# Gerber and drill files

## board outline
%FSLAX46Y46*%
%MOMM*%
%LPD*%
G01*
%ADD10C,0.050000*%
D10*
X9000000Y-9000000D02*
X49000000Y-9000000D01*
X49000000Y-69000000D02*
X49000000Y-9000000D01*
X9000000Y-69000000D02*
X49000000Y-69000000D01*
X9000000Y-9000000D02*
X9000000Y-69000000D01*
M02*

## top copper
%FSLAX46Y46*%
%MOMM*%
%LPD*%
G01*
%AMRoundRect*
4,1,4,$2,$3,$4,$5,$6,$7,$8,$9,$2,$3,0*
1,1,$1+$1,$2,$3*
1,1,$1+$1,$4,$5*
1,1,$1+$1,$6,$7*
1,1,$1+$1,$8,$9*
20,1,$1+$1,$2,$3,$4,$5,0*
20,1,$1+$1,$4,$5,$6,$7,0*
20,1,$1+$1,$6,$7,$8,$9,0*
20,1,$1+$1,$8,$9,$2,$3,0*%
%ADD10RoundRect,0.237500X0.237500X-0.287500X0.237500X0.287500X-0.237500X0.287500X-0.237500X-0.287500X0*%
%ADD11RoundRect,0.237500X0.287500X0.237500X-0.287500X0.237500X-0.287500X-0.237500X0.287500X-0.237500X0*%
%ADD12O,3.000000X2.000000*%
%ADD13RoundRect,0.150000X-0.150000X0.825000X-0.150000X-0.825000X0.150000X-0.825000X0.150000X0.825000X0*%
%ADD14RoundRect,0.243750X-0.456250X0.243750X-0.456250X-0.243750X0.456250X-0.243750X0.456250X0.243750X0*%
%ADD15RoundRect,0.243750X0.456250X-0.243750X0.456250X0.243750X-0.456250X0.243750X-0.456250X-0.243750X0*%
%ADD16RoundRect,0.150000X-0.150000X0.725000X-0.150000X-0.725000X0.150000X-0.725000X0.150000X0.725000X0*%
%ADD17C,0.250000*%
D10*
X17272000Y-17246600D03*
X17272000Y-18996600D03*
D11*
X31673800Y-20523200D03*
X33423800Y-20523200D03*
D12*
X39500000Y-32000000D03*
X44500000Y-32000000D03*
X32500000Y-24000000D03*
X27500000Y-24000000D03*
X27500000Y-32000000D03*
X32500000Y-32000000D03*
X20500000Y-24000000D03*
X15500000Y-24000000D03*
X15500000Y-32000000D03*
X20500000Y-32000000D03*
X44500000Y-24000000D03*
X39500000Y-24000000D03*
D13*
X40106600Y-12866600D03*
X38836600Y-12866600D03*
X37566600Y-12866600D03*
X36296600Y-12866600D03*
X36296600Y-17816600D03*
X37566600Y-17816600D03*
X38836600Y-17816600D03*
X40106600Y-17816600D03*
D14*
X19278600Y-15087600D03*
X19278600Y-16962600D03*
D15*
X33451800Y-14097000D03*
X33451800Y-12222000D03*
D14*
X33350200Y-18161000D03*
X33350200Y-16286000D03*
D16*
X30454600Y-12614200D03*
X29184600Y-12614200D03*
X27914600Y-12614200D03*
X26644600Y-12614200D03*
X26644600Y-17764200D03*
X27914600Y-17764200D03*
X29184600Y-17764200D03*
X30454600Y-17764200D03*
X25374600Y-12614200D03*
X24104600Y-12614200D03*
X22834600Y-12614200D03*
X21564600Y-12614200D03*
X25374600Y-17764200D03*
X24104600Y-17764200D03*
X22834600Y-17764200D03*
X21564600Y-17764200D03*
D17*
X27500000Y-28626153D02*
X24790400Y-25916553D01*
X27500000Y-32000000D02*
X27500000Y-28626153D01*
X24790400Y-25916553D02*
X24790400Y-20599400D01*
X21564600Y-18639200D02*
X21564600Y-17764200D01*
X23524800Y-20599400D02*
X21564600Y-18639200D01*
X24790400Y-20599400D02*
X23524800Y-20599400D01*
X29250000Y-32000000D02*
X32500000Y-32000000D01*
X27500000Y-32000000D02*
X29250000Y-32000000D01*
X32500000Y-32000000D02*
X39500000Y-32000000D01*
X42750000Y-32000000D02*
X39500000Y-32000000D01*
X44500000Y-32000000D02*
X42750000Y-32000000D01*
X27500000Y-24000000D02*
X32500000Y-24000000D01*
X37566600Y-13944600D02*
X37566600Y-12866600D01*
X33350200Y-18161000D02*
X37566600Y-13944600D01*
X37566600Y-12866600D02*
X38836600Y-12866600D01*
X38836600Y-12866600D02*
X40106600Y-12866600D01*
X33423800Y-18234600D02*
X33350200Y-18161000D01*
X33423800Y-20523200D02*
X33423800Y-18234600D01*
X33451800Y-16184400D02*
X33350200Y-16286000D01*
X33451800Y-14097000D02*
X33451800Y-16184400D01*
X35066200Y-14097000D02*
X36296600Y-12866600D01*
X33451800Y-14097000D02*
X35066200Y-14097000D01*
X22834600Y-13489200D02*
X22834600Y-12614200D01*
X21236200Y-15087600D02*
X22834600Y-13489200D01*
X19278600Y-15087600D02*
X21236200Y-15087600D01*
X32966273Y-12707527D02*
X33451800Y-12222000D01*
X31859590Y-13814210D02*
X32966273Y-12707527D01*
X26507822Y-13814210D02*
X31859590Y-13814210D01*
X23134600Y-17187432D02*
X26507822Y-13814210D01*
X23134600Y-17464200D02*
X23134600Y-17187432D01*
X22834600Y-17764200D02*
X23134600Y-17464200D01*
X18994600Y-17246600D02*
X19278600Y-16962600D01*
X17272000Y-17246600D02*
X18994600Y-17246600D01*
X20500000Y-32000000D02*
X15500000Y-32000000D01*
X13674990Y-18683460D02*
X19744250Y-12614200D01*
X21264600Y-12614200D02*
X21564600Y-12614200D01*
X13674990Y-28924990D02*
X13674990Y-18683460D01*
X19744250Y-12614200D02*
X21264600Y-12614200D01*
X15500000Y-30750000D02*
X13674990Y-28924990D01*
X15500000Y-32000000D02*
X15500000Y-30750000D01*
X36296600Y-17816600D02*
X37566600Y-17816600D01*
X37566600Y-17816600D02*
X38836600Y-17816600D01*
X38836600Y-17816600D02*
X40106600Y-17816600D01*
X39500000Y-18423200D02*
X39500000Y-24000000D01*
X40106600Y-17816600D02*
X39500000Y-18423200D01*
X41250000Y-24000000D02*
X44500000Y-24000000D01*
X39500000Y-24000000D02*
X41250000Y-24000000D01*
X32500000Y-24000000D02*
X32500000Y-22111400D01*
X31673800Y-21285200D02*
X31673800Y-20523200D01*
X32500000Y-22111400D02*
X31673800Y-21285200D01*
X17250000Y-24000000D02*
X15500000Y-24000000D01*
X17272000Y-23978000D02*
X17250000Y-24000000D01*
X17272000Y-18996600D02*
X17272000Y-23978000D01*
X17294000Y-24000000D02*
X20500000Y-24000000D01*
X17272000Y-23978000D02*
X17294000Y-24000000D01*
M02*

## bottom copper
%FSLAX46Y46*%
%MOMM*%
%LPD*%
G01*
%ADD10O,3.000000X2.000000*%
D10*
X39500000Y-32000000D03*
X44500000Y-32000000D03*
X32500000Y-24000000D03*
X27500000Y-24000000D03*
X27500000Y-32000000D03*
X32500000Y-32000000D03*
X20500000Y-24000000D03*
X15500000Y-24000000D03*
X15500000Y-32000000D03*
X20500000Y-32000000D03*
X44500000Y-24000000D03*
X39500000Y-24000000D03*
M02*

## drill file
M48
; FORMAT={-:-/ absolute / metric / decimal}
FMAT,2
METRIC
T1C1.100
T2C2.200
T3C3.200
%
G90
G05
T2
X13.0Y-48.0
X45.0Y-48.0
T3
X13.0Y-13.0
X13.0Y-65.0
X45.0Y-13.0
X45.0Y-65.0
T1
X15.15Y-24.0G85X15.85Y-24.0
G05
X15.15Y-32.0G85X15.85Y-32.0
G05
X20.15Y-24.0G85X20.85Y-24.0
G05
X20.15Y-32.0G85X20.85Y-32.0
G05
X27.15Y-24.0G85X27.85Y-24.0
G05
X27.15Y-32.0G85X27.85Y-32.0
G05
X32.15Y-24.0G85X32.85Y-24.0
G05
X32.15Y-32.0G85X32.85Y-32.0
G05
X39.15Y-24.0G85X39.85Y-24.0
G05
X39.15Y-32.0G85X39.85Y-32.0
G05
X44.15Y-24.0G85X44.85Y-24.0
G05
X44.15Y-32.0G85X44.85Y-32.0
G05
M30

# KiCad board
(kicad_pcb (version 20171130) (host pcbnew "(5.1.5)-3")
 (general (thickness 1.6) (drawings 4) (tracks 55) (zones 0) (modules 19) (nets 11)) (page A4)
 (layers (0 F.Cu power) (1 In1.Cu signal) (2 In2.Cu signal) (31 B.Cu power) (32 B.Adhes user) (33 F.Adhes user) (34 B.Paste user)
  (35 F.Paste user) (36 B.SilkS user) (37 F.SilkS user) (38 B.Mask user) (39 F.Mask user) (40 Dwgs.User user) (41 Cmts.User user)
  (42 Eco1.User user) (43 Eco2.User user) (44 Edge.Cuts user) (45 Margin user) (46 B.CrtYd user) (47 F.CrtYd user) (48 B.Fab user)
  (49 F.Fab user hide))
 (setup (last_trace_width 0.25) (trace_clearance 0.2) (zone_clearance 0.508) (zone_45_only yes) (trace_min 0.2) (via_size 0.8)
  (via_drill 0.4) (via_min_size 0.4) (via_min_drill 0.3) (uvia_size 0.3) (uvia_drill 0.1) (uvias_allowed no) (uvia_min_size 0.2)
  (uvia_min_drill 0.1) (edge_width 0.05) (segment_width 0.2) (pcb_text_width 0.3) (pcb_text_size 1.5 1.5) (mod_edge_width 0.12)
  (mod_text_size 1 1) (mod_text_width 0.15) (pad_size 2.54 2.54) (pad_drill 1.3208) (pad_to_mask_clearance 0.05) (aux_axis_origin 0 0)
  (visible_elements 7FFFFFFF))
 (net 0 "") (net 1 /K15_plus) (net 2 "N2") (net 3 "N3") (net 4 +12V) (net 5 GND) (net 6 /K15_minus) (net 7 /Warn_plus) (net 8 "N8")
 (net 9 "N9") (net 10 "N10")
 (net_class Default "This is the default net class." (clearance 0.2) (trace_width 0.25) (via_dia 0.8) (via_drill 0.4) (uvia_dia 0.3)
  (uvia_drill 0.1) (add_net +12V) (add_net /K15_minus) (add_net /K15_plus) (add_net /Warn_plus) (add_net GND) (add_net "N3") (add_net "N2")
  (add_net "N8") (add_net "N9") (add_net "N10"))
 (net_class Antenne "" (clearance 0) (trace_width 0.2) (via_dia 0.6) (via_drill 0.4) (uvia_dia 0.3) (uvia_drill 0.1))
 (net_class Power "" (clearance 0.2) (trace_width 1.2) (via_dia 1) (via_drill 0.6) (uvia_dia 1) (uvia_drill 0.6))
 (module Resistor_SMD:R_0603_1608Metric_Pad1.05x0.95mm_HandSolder (layer F.Cu) (at 17.272 18.1216 90)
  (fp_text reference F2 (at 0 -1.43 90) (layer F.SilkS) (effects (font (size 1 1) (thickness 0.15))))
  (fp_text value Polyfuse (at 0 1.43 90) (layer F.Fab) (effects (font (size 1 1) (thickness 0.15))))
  (pad 2 smd roundrect (at 0.875 0 90) (size 1.05 0.95) (layers F.Cu F.Paste F.Mask) (roundrect_rratio 0.25) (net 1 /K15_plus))
  (pad 1 smd roundrect (at -0.875 0 90) (size 1.05 0.95) (layers F.Cu F.Paste F.Mask) (roundrect_rratio 0.25) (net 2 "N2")))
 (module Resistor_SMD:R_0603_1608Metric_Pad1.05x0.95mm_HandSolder (layer F.Cu) (at 32.5488 20.5232 180)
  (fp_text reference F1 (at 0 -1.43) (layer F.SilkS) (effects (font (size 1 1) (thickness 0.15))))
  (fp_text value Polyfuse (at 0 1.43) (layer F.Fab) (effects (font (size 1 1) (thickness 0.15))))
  (pad 2 smd roundrect (at 0.875 0 180) (size 1.05 0.95) (layers F.Cu F.Paste F.Mask) (roundrect_rratio 0.25) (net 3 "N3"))
  (pad 1 smd roundrect (at -0.875 0 180) (size 1.05 0.95) (layers F.Cu F.Paste F.Mask) (roundrect_rratio 0.25) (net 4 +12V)))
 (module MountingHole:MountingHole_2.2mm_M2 (layer F.Cu) (at 45 48)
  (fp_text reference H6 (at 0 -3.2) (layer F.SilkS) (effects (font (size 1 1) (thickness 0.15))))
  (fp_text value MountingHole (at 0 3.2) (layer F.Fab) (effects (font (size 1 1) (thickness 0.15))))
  (pad 1 np_thru_hole circle (at 0 0) (size 2.2 2.2) (drill 2.2) (layers *.Cu *.Mask)))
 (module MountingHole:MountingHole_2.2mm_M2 (layer F.Cu) (at 13 48)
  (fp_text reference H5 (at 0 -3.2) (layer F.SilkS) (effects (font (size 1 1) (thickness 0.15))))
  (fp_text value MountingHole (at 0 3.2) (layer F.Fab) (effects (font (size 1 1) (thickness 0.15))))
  (pad 1 np_thru_hole circle (at 0 0) (size 2.2 2.2) (drill 2.2) (layers *.Cu *.Mask)))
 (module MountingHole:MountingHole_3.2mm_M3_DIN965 (layer F.Cu) (at 13 13)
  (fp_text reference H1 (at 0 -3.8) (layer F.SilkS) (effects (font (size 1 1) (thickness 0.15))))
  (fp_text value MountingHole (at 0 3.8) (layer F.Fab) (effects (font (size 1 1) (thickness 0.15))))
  (pad 1 np_thru_hole circle (at 0 0) (size 3.2 3.2) (drill 3.2) (layers *.Cu *.Mask)))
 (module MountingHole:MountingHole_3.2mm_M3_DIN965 (layer F.Cu) (at 13 65)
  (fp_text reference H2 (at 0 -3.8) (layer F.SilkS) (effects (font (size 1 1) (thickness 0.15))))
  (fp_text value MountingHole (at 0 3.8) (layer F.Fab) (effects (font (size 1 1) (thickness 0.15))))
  (pad 1 np_thru_hole circle (at 0 0) (size 3.2 3.2) (drill 3.2) (layers *.Cu *.Mask)))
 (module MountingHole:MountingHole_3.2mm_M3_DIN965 (layer F.Cu) (at 45 13)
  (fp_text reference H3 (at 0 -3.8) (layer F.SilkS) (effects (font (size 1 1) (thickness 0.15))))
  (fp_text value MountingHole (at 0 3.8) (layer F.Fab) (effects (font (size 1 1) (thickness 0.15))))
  (pad 1 np_thru_hole circle (at 0 0) (size 3.2 3.2) (drill 3.2) (layers *.Cu *.Mask)))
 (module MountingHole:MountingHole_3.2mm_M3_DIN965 (layer F.Cu) (at 45 65)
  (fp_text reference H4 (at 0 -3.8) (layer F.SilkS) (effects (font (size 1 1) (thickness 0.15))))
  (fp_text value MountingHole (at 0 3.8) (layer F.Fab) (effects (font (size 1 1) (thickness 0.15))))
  (pad 1 np_thru_hole circle (at 0 0) (size 3.2 3.2) (drill 3.2) (layers *.Cu *.Mask)))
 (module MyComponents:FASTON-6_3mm (layer F.Cu) (at 42 32)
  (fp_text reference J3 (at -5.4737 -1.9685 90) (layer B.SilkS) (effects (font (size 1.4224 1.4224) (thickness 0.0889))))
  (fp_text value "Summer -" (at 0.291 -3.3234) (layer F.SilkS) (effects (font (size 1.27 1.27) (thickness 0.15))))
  (pad 1 thru_hole oval (at -2.5 0) (size 3 2) (drill oval 1.8 1.1) (layers *.Cu F.Paste F.SilkS F.Mask) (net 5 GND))
  (pad 1 thru_hole oval (at 2.5 0) (size 3 2) (drill oval 1.8 1.1) (layers *.Cu F.Paste F.SilkS F.Mask) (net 5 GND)))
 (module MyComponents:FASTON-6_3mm (layer F.Cu) (at 30 24)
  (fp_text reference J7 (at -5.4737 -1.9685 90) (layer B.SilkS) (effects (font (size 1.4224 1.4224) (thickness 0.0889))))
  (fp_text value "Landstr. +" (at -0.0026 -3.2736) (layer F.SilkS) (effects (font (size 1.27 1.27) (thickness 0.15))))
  (pad 1 thru_hole oval (at 2.5 0) (size 3 2) (drill oval 1.8 1.1) (layers *.Cu F.Paste F.SilkS F.Mask) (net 3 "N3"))
  (pad 1 thru_hole oval (at -2.5 0) (size 3 2) (drill oval 1.8 1.1) (layers *.Cu F.Paste F.SilkS F.Mask) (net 3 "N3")))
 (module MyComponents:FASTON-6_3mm (layer F.Cu) (at 30 32)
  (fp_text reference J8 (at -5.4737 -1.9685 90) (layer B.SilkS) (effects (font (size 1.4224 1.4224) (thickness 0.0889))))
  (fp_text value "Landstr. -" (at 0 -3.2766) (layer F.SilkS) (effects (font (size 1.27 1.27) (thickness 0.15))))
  (pad 1 thru_hole oval (at -2.5 0) (size 3 2) (drill oval 1.8 1.1) (layers *.Cu F.Paste F.SilkS F.Mask) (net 5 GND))
  (pad 1 thru_hole oval (at 2.5 0) (size 3 2) (drill oval 1.8 1.1) (layers *.Cu F.Paste F.SilkS F.Mask) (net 5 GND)))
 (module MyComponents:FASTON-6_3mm (layer F.Cu) (at 18 24)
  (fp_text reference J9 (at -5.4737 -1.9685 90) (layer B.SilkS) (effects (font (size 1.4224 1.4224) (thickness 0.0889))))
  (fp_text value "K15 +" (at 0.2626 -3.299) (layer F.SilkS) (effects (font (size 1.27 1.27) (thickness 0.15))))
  (pad 1 thru_hole oval (at 2.5 0) (size 3 2) (drill oval 1.8 1.1) (layers *.Cu F.Paste F.SilkS F.Mask) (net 2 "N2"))
  (pad 1 thru_hole oval (at -2.5 0) (size 3 2) (drill oval 1.8 1.1) (layers *.Cu F.Paste F.SilkS F.Mask) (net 2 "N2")))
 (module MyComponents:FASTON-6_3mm (layer F.Cu) (at 18 32)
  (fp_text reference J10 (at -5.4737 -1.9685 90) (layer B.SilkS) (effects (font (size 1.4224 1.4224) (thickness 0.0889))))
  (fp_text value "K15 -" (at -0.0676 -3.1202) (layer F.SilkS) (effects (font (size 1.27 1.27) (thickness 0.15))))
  (pad 1 thru_hole oval (at -2.5 0) (size 3 2) (drill oval 1.8 1.1) (layers *.Cu F.Paste F.SilkS F.Mask) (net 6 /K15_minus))
  (pad 1 thru_hole oval (at 2.5 0) (size 3 2) (drill oval 1.8 1.1) (layers *.Cu F.Paste F.SilkS F.Mask) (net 6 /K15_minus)))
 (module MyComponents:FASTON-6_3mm (layer F.Cu) (at 42 24)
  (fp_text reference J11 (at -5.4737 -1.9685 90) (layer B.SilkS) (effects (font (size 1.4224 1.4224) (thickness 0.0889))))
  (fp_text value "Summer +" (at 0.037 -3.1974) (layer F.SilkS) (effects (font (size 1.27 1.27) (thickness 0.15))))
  (pad 1 thru_hole oval (at 2.5 0) (size 3 2) (drill oval 1.8 1.1) (layers *.Cu F.Paste F.SilkS F.Mask) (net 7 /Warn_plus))
  (pad 1 thru_hole oval (at -2.5 0) (size 3 2) (drill oval 1.8 1.1) (layers *.Cu F.Paste F.SilkS F.Mask) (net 7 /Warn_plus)))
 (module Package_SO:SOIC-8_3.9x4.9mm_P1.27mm (layer F.Cu) (at 38.2016 15.3416 270)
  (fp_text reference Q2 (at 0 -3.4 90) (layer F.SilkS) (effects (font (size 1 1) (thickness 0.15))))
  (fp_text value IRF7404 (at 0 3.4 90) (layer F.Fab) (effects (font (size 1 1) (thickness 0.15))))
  (pad 1 smd roundrect (at -2.475 -1.905 270) (size 1.95 0.6) (layers F.Cu F.Paste F.Mask) (roundrect_rratio 0.25) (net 4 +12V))
  (pad 2 smd roundrect (at -2.475 -0.635 270) (size 1.95 0.6) (layers F.Cu F.Paste F.Mask) (roundrect_rratio 0.25) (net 4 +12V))
  (pad 3 smd roundrect (at -2.475 0.635 270) (size 1.95 0.6) (layers F.Cu F.Paste F.Mask) (roundrect_rratio 0.25) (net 4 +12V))
  (pad 4 smd roundrect (at -2.475 1.905 270) (size 1.95 0.6) (layers F.Cu F.Paste F.Mask) (roundrect_rratio 0.25) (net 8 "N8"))
  (pad 5 smd roundrect (at 2.475 1.905 270) (size 1.95 0.6) (layers F.Cu F.Paste F.Mask) (roundrect_rratio 0.25) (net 7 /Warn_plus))
  (pad 6 smd roundrect (at 2.475 0.635 270) (size 1.95 0.6) (layers F.Cu F.Paste F.Mask) (roundrect_rratio 0.25) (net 7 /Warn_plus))
  (pad 7 smd roundrect (at 2.475 -0.635 270) (size 1.95 0.6) (layers F.Cu F.Paste F.Mask) (roundrect_rratio 0.25) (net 7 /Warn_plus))
  (pad 8 smd roundrect (at 2.475 -1.905 270) (size 1.95 0.6) (layers F.Cu F.Paste F.Mask) (roundrect_rratio 0.25) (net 7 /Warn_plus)))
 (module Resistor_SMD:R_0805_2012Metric (layer F.Cu) (at 19.2786 16.0251 270)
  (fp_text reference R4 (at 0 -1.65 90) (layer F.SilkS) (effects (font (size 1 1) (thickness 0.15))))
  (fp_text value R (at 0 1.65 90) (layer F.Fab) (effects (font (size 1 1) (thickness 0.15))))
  (pad 1 smd roundrect (at -0.9375 0 270) (size 0.975 1.4) (layers F.Cu F.Paste F.Mask) (roundrect_rratio 0.25) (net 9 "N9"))
  (pad 2 smd roundrect (at 0.9375 0 270) (size 0.975 1.4) (layers F.Cu F.Paste F.Mask) (roundrect_rratio 0.25) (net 1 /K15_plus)))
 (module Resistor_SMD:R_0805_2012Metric (layer F.Cu) (at 33.4518 13.1595 90)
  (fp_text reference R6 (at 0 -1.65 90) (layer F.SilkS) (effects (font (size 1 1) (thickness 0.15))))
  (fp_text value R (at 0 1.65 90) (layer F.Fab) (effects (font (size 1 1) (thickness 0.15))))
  (pad 1 smd roundrect (at -0.9375 0 90) (size 0.975 1.4) (layers F.Cu F.Paste F.Mask) (roundrect_rratio 0.25) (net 8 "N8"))
  (pad 2 smd roundrect (at 0.9375 0 90) (size 0.975 1.4) (layers F.Cu F.Paste F.Mask) (roundrect_rratio 0.25) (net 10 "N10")))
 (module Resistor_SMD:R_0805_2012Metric (layer F.Cu) (at 33.3502 17.2235 270)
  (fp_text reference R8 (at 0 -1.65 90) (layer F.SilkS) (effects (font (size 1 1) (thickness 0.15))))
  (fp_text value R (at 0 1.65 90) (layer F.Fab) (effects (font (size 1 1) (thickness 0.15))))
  (pad 2 smd roundrect (at 0.9375 0 270) (size 0.975 1.4) (layers F.Cu F.Paste F.Mask) (roundrect_rratio 0.25) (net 4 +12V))
  (pad 1 smd roundrect (at -0.9375 0 270) (size 0.975 1.4) (layers F.Cu F.Paste F.Mask) (roundrect_rratio 0.25) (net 8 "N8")))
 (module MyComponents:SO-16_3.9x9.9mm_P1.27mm (layer F.Cu) (at 28.5496 15.1892 270)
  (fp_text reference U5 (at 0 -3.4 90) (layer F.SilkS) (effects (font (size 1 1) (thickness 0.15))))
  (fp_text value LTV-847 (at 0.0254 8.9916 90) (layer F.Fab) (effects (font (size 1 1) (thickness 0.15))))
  (pad 1 smd roundrect (at -2.575 -1.905 270) (size 1.75 0.6) (layers F.Cu F.Paste F.Mask) (roundrect_rratio 0.25))
  (pad 2 smd roundrect (at -2.575 -0.635 270) (size 1.75 0.6) (layers F.Cu F.Paste F.Mask) (roundrect_rratio 0.25))
  (pad 3 smd roundrect (at -2.575 0.635 270) (size 1.75 0.6) (layers F.Cu F.Paste F.Mask) (roundrect_rratio 0.25))
  (pad 4 smd roundrect (at -2.575 1.905 270) (size 1.75 0.6) (layers F.Cu F.Paste F.Mask) (roundrect_rratio 0.25))
  (pad 13 smd roundrect (at 2.575 1.905 270) (size 1.75 0.6) (layers F.Cu F.Paste F.Mask) (roundrect_rratio 0.25))
  (pad 14 smd roundrect (at 2.575 0.635 270) (size 1.75 0.6) (layers F.Cu F.Paste F.Mask) (roundrect_rratio 0.25))
  (pad 15 smd roundrect (at 2.575 -0.635 270) (size 1.75 0.6) (layers F.Cu F.Paste F.Mask) (roundrect_rratio 0.25))
  (pad 16 smd roundrect (at 2.575 -1.905 270) (size 1.75 0.6) (layers F.Cu F.Paste F.Mask) (roundrect_rratio 0.25))
  (pad 5 smd roundrect (at -2.575 3.175 270) (size 1.75 0.6) (layers F.Cu F.Paste F.Mask) (roundrect_rratio 0.25))
  (pad 6 smd roundrect (at -2.575 4.445 270) (size 1.75 0.6) (layers F.Cu F.Paste F.Mask) (roundrect_rratio 0.25))
  (pad 7 smd roundrect (at -2.575 5.715 270) (size 1.75 0.6) (layers F.Cu F.Paste F.Mask) (roundrect_rratio 0.25) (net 9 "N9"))
  (pad 8 smd roundrect (at -2.575 6.985 270) (size 1.75 0.6) (layers F.Cu F.Paste F.Mask) (roundrect_rratio 0.25) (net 6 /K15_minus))
  (pad 12 smd roundrect (at 2.575 3.175 270) (size 1.75 0.6) (layers F.Cu F.Paste F.Mask) (roundrect_rratio 0.25))
  (pad 11 smd roundrect (at 2.575 4.445 270) (size 1.75 0.6) (layers F.Cu F.Paste F.Mask) (roundrect_rratio 0.25))
  (pad 10 smd roundrect (at 2.575 5.715 270) (size 1.75 0.6) (layers F.Cu F.Paste F.Mask) (roundrect_rratio 0.25) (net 10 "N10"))
  (pad 9 smd roundrect (at 2.575 6.985 270) (size 1.75 0.6) (layers F.Cu F.Paste F.Mask) (roundrect_rratio 0.25) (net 5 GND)))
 (gr_line (start 9 9) (end 49 9) (layer Edge.Cuts) (width 0.05))
 (gr_line (start 49 69) (end 49 9) (layer Edge.Cuts) (width 0.05))
 (gr_line (start 9 69) (end 49 69) (layer Edge.Cuts) (width 0.05))
 (gr_line (start 9 9) (end 9 69) (layer Edge.Cuts) (width 0.05))
 (segment (start 27.5 28.626153) (end 24.7904 25.916553) (width 0.25) (layer F.Cu) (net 5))
 (segment (start 27.5 32) (end 27.5 28.626153) (width 0.25) (layer F.Cu) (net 5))
 (segment (start 24.7904 25.916553) (end 24.7904 20.5994) (width 0.25) (layer F.Cu) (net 5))
 (segment (start 21.5646 18.6392) (end 21.5646 17.7642) (width 0.25) (layer F.Cu) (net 5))
 (segment (start 23.5248 20.5994) (end 21.5646 18.6392) (width 0.25) (layer F.Cu) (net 5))
 (segment (start 24.7904 20.5994) (end 23.5248 20.5994) (width 0.25) (layer F.Cu) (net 5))
 (segment (start 29.25 32) (end 32.5 32) (width 0.25) (layer F.Cu) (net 5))
 (segment (start 27.5 32) (end 29.25 32) (width 0.25) (layer F.Cu) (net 5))
 (segment (start 32.5 32) (end 39.5 32) (width 0.25) (layer F.Cu) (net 5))
 (segment (start 42.75 32) (end 39.5 32) (width 0.25) (layer F.Cu) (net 5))
 (segment (start 44.5 32) (end 42.75 32) (width 0.25) (layer F.Cu) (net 5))
 (segment (start 27.5 24) (end 32.5 24) (width 0.25) (layer F.Cu) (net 3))
 (segment (start 37.5666 13.9446) (end 37.5666 12.8666) (width 0.25) (layer F.Cu) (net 4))
 (segment (start 33.3502 18.161) (end 37.5666 13.9446) (width 0.25) (layer F.Cu) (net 4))
 (segment (start 37.5666 12.8666) (end 38.8366 12.8666) (width 0.25) (layer F.Cu) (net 4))
 (segment (start 38.8366 12.8666) (end 40.1066 12.8666) (width 0.25) (layer F.Cu) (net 4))
 (segment (start 33.4238 18.2346) (end 33.3502 18.161) (width 0.25) (layer F.Cu) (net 4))
 (segment (start 33.4238 20.5232) (end 33.4238 18.2346) (width 0.25) (layer F.Cu) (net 4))
 (segment (start 33.4518 16.1844) (end 33.3502 16.286) (width 0.25) (layer F.Cu) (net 8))
 (segment (start 33.4518 14.097) (end 33.4518 16.1844) (width 0.25) (layer F.Cu) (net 8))
 (segment (start 35.0662 14.097) (end 36.2966 12.8666) (width 0.25) (layer F.Cu) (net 8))
 (segment (start 33.4518 14.097) (end 35.0662 14.097) (width 0.25) (layer F.Cu) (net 8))
 (segment (start 22.8346 13.4892) (end 22.8346 12.6142) (width 0.25) (layer F.Cu) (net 9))
 (segment (start 21.2362 15.0876) (end 22.8346 13.4892) (width 0.25) (layer F.Cu) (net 9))
 (segment (start 19.2786 15.0876) (end 21.2362 15.0876) (width 0.25) (layer F.Cu) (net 9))
 (segment (start 32.966273 12.707527) (end 33.4518 12.222) (width 0.25) (layer F.Cu) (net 10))
 (segment (start 31.85959 13.81421) (end 32.966273 12.707527) (width 0.25) (layer F.Cu) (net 10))
 (segment (start 26.507822 13.81421) (end 31.85959 13.81421) (width 0.25) (layer F.Cu) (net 10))
 (segment (start 23.1346 17.187432) (end 26.507822 13.81421) (width 0.25) (layer F.Cu) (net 10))
 (segment (start 23.1346 17.4642) (end 23.1346 17.187432) (width 0.25) (layer F.Cu) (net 10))
 (segment (start 22.8346 17.7642) (end 23.1346 17.4642) (width 0.25) (layer F.Cu) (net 10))
 (segment (start 18.9946 17.2466) (end 19.2786 16.9626) (width 0.25) (layer F.Cu) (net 1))
 (segment (start 17.272 17.2466) (end 18.9946 17.2466) (width 0.25) (layer F.Cu) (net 1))
 (segment (start 20.5 32) (end 15.5 32) (width 0.25) (layer F.Cu) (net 6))
 (segment (start 13.67499 18.68346) (end 19.74425 12.6142) (width 0.25) (layer F.Cu) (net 6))
 (segment (start 21.2646 12.6142) (end 21.5646 12.6142) (width 0.25) (layer F.Cu) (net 6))
 (segment (start 13.67499 28.92499) (end 13.67499 18.68346) (width 0.25) (layer F.Cu) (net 6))
 (segment (start 19.74425 12.6142) (end 21.2646 12.6142) (width 0.25) (layer F.Cu) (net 6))
 (segment (start 15.5 30.75) (end 13.67499 28.92499) (width 0.25) (layer F.Cu) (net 6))
 (segment (start 15.5 32) (end 15.5 30.75) (width 0.25) (layer F.Cu) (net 6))
 (segment (start 36.2966 17.8166) (end 37.5666 17.8166) (width 0.25) (layer F.Cu) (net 7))
 (segment (start 37.5666 17.8166) (end 38.8366 17.8166) (width 0.25) (layer F.Cu) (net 7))
 (segment (start 38.8366 17.8166) (end 40.1066 17.8166) (width 0.25) (layer F.Cu) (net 7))
 (segment (start 39.5 18.4232) (end 39.5 24) (width 0.25) (layer F.Cu) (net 7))
 (segment (start 40.1066 17.8166) (end 39.5 18.4232) (width 0.25) (layer F.Cu) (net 7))
 (segment (start 41.25 24) (end 44.5 24) (width 0.25) (layer F.Cu) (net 7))
 (segment (start 39.5 24) (end 41.25 24) (width 0.25) (layer F.Cu) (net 7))
 (segment (start 32.5 24) (end 32.5 22.1114) (width 0.25) (layer F.Cu) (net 3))
 (segment (start 31.6738 21.2852) (end 31.6738 20.5232) (width 0.25) (layer F.Cu) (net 3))
 (segment (start 32.5 22.1114) (end 31.6738 21.2852) (width 0.25) (layer F.Cu) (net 3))
 (segment (start 17.25 24) (end 15.5 24) (width 0.25) (layer F.Cu) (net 2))
 (segment (start 17.272 23.978) (end 17.25 24) (width 0.25) (layer F.Cu) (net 2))
 (segment (start 17.272 18.9966) (end 17.272 23.978) (width 0.25) (layer F.Cu) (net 2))
 (segment (start 17.294 24) (end 20.5 24) (width 0.25) (layer F.Cu) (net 2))
 (segment (start 17.272 23.978) (end 17.294 24) (width 0.25) (layer F.Cu) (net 2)))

